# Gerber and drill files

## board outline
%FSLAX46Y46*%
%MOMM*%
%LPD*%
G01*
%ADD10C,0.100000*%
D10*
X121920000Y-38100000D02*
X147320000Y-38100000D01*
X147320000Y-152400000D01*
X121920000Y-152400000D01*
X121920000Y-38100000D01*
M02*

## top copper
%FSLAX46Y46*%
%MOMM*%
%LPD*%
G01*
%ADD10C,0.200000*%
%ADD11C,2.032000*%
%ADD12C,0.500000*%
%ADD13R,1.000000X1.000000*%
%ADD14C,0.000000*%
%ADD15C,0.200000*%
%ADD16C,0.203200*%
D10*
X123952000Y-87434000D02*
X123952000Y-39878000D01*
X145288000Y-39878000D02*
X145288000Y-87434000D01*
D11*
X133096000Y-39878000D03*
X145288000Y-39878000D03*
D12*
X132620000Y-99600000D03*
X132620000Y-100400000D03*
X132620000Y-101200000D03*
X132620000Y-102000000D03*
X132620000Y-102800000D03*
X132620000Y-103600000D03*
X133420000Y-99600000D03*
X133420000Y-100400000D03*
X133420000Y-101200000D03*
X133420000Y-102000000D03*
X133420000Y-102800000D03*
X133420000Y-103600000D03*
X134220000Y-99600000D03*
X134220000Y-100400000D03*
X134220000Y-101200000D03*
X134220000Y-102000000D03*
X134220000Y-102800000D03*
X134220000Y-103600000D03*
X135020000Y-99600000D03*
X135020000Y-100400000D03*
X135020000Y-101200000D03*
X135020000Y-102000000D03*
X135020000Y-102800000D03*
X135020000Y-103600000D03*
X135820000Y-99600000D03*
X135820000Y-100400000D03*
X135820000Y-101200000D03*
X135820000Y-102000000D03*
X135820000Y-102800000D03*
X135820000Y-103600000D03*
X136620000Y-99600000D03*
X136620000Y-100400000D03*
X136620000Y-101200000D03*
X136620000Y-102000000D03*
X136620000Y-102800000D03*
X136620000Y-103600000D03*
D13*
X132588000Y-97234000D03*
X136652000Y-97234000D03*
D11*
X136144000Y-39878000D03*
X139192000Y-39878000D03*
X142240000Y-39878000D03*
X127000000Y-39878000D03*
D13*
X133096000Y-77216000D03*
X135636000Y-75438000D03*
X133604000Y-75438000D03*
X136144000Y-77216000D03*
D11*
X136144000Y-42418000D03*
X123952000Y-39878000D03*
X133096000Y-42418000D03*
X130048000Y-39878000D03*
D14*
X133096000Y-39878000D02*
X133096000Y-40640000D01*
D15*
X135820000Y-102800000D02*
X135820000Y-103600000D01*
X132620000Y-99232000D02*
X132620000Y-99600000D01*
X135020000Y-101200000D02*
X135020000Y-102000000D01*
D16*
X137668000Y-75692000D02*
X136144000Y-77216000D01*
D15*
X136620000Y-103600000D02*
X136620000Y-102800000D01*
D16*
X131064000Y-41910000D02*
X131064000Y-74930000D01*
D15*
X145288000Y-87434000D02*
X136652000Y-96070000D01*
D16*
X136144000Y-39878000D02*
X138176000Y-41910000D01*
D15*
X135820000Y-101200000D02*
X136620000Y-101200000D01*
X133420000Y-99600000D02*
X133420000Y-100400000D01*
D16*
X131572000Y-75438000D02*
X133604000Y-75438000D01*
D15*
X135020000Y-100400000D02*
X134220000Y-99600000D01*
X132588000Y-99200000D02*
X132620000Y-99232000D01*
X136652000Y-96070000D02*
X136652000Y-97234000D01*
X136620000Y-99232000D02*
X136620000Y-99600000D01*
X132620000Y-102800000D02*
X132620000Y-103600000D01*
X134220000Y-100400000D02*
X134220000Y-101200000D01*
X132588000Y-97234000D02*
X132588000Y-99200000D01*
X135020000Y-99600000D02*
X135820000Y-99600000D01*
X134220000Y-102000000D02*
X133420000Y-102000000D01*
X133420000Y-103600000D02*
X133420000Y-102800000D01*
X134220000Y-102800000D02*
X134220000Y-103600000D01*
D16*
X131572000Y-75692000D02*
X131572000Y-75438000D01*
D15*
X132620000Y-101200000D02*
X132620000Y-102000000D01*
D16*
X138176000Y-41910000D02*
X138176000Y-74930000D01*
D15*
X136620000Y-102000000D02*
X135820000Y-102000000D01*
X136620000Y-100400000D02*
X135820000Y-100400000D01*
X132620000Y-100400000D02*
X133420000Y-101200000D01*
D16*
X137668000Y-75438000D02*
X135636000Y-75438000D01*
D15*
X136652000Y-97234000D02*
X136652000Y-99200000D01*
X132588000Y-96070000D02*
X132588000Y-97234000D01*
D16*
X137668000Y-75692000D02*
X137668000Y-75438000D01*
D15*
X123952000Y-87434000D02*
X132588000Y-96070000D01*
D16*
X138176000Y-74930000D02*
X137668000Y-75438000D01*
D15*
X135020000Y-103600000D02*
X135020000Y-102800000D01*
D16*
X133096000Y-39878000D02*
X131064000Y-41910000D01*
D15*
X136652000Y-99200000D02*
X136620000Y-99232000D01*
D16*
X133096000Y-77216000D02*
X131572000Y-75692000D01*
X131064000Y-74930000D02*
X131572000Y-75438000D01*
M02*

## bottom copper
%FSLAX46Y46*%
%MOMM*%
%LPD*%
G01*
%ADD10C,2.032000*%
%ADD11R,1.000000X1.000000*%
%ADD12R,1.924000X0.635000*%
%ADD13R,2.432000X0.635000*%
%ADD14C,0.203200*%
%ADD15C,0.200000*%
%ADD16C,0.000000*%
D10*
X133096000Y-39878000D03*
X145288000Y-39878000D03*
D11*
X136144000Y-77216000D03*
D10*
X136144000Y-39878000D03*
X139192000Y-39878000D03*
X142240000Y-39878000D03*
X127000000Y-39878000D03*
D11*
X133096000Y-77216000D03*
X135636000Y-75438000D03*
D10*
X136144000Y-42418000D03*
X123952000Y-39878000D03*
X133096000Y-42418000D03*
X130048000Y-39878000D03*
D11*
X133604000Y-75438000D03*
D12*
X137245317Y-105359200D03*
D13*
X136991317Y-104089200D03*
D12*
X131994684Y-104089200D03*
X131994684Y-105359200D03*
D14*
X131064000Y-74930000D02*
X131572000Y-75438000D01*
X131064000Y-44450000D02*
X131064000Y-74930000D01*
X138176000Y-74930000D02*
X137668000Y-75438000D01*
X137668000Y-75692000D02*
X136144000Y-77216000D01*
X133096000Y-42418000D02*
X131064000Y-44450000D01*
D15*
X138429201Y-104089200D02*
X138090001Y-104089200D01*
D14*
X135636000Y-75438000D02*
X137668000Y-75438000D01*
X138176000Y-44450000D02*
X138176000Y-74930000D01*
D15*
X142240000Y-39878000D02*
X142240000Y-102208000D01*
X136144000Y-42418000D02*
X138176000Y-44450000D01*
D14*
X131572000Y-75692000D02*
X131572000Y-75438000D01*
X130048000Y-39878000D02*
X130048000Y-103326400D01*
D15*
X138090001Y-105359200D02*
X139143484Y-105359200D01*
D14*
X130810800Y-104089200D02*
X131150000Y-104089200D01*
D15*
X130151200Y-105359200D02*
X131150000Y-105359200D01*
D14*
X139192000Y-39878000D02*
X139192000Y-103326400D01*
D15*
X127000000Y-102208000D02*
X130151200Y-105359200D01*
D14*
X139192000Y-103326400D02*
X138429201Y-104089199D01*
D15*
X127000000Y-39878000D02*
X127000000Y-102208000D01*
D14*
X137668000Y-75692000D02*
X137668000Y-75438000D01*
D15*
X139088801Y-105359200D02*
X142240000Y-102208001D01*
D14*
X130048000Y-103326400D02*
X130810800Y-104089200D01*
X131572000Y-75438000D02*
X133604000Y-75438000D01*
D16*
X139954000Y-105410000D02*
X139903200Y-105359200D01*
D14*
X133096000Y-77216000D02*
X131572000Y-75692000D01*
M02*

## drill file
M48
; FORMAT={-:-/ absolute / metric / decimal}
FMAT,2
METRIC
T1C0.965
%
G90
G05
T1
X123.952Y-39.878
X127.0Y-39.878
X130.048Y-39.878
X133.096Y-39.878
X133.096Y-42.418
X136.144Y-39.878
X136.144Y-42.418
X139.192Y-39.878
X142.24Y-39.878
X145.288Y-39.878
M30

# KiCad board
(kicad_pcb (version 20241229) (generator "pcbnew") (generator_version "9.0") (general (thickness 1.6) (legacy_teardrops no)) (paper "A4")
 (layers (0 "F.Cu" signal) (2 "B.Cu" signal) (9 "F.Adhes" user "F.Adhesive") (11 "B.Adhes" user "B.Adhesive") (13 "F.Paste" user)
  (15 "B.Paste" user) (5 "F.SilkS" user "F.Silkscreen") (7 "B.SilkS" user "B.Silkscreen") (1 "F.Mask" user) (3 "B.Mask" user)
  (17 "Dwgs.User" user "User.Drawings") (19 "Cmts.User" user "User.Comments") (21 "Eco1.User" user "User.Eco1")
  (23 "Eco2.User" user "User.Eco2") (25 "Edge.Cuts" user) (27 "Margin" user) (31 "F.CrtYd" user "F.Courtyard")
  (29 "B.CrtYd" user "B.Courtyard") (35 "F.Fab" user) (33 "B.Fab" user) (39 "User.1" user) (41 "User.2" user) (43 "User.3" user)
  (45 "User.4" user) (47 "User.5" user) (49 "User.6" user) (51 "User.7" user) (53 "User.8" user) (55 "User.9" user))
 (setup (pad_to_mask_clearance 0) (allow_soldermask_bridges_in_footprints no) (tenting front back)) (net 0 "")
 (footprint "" (layer "F.Cu") (at 133.096 52.578)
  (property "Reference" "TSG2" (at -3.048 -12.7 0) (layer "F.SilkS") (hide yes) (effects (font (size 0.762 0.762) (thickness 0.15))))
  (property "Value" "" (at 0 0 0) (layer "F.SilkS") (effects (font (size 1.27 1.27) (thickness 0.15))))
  (pad "1" thru_hole circle (at 0 -12.7) (size 2.032 2.032) (drill 0.9652) (layers "*.Cu" "*.Mask") (remove_unused_layers no)))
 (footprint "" (layer "F.Cu") (at 145.796 39.878)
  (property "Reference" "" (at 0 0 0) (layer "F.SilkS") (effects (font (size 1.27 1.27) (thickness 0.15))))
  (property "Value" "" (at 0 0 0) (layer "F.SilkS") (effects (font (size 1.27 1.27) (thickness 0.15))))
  (pad "1" thru_hole circle (at -0.508 0) (size 2.032 2.032) (drill 0.9652) (layers "*.Cu" "*.Mask") (remove_unused_layers no)))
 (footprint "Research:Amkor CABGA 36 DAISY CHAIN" (layer "F.Cu") (at 134.62 92.535)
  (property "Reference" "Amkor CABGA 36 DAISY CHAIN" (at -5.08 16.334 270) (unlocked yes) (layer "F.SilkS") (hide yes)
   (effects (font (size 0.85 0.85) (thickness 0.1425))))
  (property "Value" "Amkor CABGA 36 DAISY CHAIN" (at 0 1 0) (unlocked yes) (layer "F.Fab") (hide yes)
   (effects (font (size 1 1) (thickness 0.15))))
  (pad "1" smd circle (at -2 7.065) (size 0.5 0.5) (layers "F.Cu" "F.Mask"))
  (pad "1" smd circle (at -2 7.865) (size 0.5 0.5) (layers "F.Cu" "F.Mask"))
  (pad "1" smd circle (at -2 8.665) (size 0.5 0.5) (layers "F.Cu" "F.Mask"))
  (pad "1" smd circle (at -2 9.465) (size 0.5 0.5) (layers "F.Cu" "F.Mask"))
  (pad "1" smd circle (at -2 10.265) (size 0.5 0.5) (layers "F.Cu" "F.Mask"))
  (pad "1" smd circle (at -2 11.065) (size 0.5 0.5) (layers "F.Cu" "F.Mask"))
  (pad "1" smd circle (at -1.2 7.065) (size 0.5 0.5) (layers "F.Cu" "F.Mask"))
  (pad "1" smd circle (at -1.2 7.865) (size 0.5 0.5) (layers "F.Cu" "F.Mask"))
  (pad "1" smd circle (at -1.2 8.665) (size 0.5 0.5) (layers "F.Cu" "F.Mask"))
  (pad "1" smd circle (at -1.2 9.465) (size 0.5 0.5) (layers "F.Cu" "F.Mask"))
  (pad "1" smd circle (at -1.2 10.265) (size 0.5 0.5) (layers "F.Cu" "F.Mask"))
  (pad "1" smd circle (at -1.2 11.065) (size 0.5 0.5) (layers "F.Cu" "F.Mask"))
  (pad "1" smd circle (at -0.4 7.065) (size 0.5 0.5) (layers "F.Cu" "F.Mask"))
  (pad "1" smd circle (at -0.4 7.865) (size 0.5 0.5) (layers "F.Cu" "F.Mask"))
  (pad "1" smd circle (at -0.4 8.665) (size 0.5 0.5) (layers "F.Cu" "F.Mask"))
  (pad "1" smd circle (at -0.4 9.465) (size 0.5 0.5) (layers "F.Cu" "F.Mask"))
  (pad "1" smd circle (at -0.4 10.265) (size 0.5 0.5) (layers "F.Cu" "F.Mask"))
  (pad "1" smd circle (at -0.4 11.065) (size 0.5 0.5) (layers "F.Cu" "F.Mask"))
  (pad "1" smd circle (at 0.4 7.065) (size 0.5 0.5) (layers "F.Cu" "F.Mask"))
  (pad "1" smd circle (at 0.4 7.865) (size 0.5 0.5) (layers "F.Cu" "F.Mask"))
  (pad "1" smd circle (at 0.4 8.665) (size 0.5 0.5) (layers "F.Cu" "F.Mask"))
  (pad "1" smd circle (at 0.4 9.465) (size 0.5 0.5) (layers "F.Cu" "F.Mask"))
  (pad "1" smd circle (at 0.4 10.265) (size 0.5 0.5) (layers "F.Cu" "F.Mask"))
  (pad "1" smd circle (at 0.4 11.065) (size 0.5 0.5) (layers "F.Cu" "F.Mask"))
  (pad "1" smd circle (at 1.2 7.065) (size 0.5 0.5) (layers "F.Cu" "F.Mask"))
  (pad "1" smd circle (at 1.2 7.865) (size 0.5 0.5) (layers "F.Cu" "F.Mask"))
  (pad "1" smd circle (at 1.2 8.665) (size 0.5 0.5) (layers "F.Cu" "F.Mask"))
  (pad "1" smd circle (at 1.2 9.465) (size 0.5 0.5) (layers "F.Cu" "F.Mask"))
  (pad "1" smd circle (at 1.2 10.265) (size 0.5 0.5) (layers "F.Cu" "F.Mask"))
  (pad "1" smd circle (at 1.2 11.065) (size 0.5 0.5) (layers "F.Cu" "F.Mask"))
  (pad "1" smd circle (at 2 7.065) (size 0.5 0.5) (layers "F.Cu" "F.Mask"))
  (pad "1" smd circle (at 2 7.865) (size 0.5 0.5) (layers "F.Cu" "F.Mask"))
  (pad "1" smd circle (at 2 8.665) (size 0.5 0.5) (layers "F.Cu" "F.Mask"))
  (pad "1" smd circle (at 2 9.465) (size 0.5 0.5) (layers "F.Cu" "F.Mask"))
  (pad "1" smd circle (at 2 10.265) (size 0.5 0.5) (layers "F.Cu" "F.Mask"))
  (pad "1" smd circle (at 2 11.065) (size 0.5 0.5) (layers "F.Cu" "F.Mask"))
  (pad "2" smd rect (at -2.032 4.699) (size 1 1) (layers "F.Cu" "F.Mask"))
  (pad "3" smd rect (at 2.032 4.699) (size 1 1) (layers "F.Cu" "F.Mask")))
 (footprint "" (layer "F.Cu") (at 136.144 77.216)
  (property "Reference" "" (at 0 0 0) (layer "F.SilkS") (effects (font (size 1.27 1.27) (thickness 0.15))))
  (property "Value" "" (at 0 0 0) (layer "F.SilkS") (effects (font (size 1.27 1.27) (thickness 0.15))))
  (pad "1" smd rect (at 0 0 180) (size 1 1) (layers "B.Cu" "B.Mask")))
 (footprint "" (layer "F.Cu") (at 135.89 52.578)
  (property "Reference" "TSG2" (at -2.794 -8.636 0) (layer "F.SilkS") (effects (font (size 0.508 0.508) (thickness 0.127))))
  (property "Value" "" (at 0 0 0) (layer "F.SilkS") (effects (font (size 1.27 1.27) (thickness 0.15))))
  (pad "1" thru_hole circle (at 0.254 -12.7) (size 2.032 2.032) (drill 0.9652) (layers "*.Cu" "*.Mask") (remove_unused_layers no)))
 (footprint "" (layer "F.Cu") (at 139.192 39.878)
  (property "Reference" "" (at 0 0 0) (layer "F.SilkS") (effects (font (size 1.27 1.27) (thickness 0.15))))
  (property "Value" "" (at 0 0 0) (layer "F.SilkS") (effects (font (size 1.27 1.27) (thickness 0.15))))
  (pad "1" thru_hole circle (at 0 0) (size 2.032 2.032) (drill 0.9652) (layers "*.Cu" "*.Mask") (remove_unused_layers no)))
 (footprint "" (layer "F.Cu") (at 142.494 39.878)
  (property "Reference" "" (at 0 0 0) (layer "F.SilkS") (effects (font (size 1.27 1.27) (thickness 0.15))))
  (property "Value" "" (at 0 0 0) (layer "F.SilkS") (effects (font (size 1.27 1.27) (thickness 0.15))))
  (pad "1" thru_hole circle (at -0.254 0) (size 2.032 2.032) (drill 0.9652) (layers "*.Cu" "*.Mask") (remove_unused_layers no)))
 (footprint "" (layer "F.Cu") (at 127 39.878)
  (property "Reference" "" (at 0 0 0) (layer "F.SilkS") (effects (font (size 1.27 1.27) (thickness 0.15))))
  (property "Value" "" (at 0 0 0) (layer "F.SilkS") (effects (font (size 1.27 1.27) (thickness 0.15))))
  (pad "1" thru_hole circle (at 0 0) (size 2.032 2.032) (drill 0.9652) (layers "*.Cu" "*.Mask") (remove_unused_layers no)))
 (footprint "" (layer "F.Cu") (at 133.096 77.216)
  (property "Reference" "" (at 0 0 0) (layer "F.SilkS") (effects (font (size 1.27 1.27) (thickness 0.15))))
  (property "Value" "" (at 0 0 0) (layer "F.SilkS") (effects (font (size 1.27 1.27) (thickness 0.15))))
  (pad "1" smd rect (at 0 0) (size 1 1) (layers "F.Cu" "F.Mask")))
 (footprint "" (layer "F.Cu") (at 133.096 77.216)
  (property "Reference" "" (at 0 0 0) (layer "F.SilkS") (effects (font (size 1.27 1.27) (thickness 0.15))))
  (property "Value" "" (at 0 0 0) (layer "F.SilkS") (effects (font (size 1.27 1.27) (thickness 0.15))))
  (pad "1" smd rect (at 0 0 180) (size 1 1) (layers "B.Cu" "B.Mask")))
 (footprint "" (layer "F.Cu") (at 135.636 75.438)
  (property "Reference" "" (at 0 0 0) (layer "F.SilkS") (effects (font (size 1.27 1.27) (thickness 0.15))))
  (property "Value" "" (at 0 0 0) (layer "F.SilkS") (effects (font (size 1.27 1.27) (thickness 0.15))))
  (pad "1" smd rect (at 0 0) (size 1 1) (layers "F.Cu" "F.Mask")))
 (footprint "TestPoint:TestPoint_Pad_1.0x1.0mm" (layer "F.Cu") (at 133.604 75.438)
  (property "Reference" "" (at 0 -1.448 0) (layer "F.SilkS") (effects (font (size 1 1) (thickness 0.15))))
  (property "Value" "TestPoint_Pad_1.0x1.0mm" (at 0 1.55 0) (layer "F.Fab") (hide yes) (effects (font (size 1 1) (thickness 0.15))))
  (pad "1" smd rect (at 0 0) (size 1 1) (layers "F.Cu" "F.Mask")))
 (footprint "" (layer "F.Cu") (at 136.144 77.216)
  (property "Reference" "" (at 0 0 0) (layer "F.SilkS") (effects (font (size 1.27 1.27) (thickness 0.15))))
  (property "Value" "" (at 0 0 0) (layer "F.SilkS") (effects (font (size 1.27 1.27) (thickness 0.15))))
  (pad "1" smd rect (at 0 0) (size 1 1) (layers "F.Cu" "F.Mask")))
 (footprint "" (layer "F.Cu") (at 135.636 75.438)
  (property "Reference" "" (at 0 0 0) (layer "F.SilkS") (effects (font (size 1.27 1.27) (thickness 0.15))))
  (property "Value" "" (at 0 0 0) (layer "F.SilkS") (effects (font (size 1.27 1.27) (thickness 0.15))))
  (pad "1" smd rect (at 0 0 180) (size 1 1) (layers "B.Cu" "B.Mask")))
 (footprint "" (layer "F.Cu") (at 135.89 55.118)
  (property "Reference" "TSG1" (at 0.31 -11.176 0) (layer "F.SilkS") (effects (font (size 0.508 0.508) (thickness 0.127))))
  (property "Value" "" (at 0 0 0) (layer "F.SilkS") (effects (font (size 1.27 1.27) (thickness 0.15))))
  (pad "1" thru_hole circle (at 0.254 -12.7) (size 2.032 2.032) (drill 0.9652) (layers "*.Cu" "*.Mask") (remove_unused_layers no)))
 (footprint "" (layer "F.Cu") (at 123.952 39.878)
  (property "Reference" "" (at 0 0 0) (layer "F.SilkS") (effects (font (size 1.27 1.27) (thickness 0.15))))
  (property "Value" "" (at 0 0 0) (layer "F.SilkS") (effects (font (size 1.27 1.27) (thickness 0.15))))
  (pad "1" thru_hole circle (at 0 0) (size 2.032 2.032) (drill 0.9652) (layers "*.Cu" "*.Mask") (remove_unused_layers no)))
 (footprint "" (layer "F.Cu") (at 133.096 55.118)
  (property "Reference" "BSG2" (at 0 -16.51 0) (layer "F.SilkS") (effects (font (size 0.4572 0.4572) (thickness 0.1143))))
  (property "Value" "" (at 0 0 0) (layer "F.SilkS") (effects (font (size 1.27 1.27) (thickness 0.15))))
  (pad "1" thru_hole circle (at 0 -12.7) (size 2.032 2.032) (drill 0.9652) (layers "*.Cu" "*.Mask") (remove_unused_layers no)))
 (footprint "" (layer "B.Cu") (at 130.048 39.878)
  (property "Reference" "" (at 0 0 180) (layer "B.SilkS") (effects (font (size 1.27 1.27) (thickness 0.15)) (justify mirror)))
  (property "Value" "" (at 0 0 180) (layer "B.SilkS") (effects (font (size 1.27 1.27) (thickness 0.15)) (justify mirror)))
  (pad "1" thru_hole circle (at 0 0) (size 2.032 2.032) (drill 0.9652) (layers "*.Cu" "*.Mask") (remove_unused_layers no)))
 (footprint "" (layer "B.Cu") (at 133.604 75.438 180)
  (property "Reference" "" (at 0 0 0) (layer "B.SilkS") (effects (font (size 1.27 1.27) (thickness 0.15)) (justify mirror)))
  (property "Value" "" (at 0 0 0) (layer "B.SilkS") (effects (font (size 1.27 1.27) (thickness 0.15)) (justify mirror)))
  (pad "1" smd rect (at 0 0 180) (size 1 1) (layers "B.Cu" "B.Mask")))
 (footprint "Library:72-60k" (layer "B.Cu") (at 132.873329 109.1692 180)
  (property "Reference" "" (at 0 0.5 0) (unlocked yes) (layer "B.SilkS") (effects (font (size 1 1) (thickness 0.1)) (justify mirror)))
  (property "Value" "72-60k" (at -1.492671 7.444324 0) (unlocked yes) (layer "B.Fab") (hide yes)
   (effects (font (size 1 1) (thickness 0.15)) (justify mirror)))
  (pad "1" smd rect (at -4.371988 3.81) (size 1.924 0.635) (layers "B.Cu" "B.Mask"))
  (pad "2" smd rect (at -4.117988 5.08) (size 2.432 0.635) (layers "B.Cu" "B.Mask"))
  (pad "3" smd rect (at 0.878645 5.08) (size 1.924 0.635) (layers "B.Cu" "B.Mask"))
  (pad "4" smd rect (at 0.878645 3.81) (size 1.924 0.635) (layers "B.Cu" "B.Mask")))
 (gr_line (start 123.952 87.434) (end 123.952 39.878) (stroke (width 0.2) (type solid)) (layer "F.Cu"))
 (gr_line (start 145.288 39.878) (end 145.288 87.434) (stroke (width 0.2) (type solid)) (layer "F.Cu"))
 (gr_rect (start 121.92 38.1) (end 147.32 152.4) (stroke (width 0.1) (type solid)) (fill no) (layer "Edge.Cuts"))
 (segment (start 133.096 39.878) (end 133.096 40.64) (width 0) (layer "F.Cu") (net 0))
 (segment (start 135.82 102.8) (end 135.82 103.6) (width 0.2) (layer "F.Cu") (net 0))
 (segment (start 132.62 99.232) (end 132.62 99.6) (width 0.2) (layer "F.Cu") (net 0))
 (segment (start 135.02 101.2) (end 135.02 102) (width 0.2) (layer "F.Cu") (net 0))
 (segment (start 137.668 75.692) (end 136.144 77.216) (width 0.2032) (layer "F.Cu") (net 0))
 (segment (start 136.62 103.6) (end 136.62 102.8) (width 0.2) (layer "F.Cu") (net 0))
 (segment (start 131.064 41.91) (end 131.064 74.93) (width 0.2032) (layer "F.Cu") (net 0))
 (segment (start 145.288 87.434) (end 136.652 96.07) (width 0.2) (layer "F.Cu") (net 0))
 (segment (start 136.144 39.878) (end 138.176 41.91) (width 0.2032) (layer "F.Cu") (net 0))
 (segment (start 135.82 101.2) (end 136.62 101.2) (width 0.2) (layer "F.Cu") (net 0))
 (segment (start 133.42 99.6) (end 133.42 100.4) (width 0.2) (layer "F.Cu") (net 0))
 (segment (start 131.572 75.438) (end 133.604 75.438) (width 0.2032) (layer "F.Cu") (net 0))
 (segment (start 135.02 100.4) (end 134.22 99.6) (width 0.2) (layer "F.Cu") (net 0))
 (segment (start 132.588 99.2) (end 132.62 99.232) (width 0.2) (layer "F.Cu") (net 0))
 (segment (start 136.652 96.07) (end 136.652 97.234) (width 0.2) (layer "F.Cu") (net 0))
 (segment (start 136.62 99.232) (end 136.62 99.6) (width 0.2) (layer "F.Cu") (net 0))
 (segment (start 132.62 102.8) (end 132.62 103.6) (width 0.2) (layer "F.Cu") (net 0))
 (segment (start 134.22 100.4) (end 134.22 101.2) (width 0.2) (layer "F.Cu") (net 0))
 (segment (start 132.588 97.234) (end 132.588 99.2) (width 0.2) (layer "F.Cu") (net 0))
 (segment (start 135.02 99.6) (end 135.82 99.6) (width 0.2) (layer "F.Cu") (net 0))
 (segment (start 134.22 102) (end 133.42 102) (width 0.2) (layer "F.Cu") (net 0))
 (segment (start 133.42 103.6) (end 133.42 102.8) (width 0.2) (layer "F.Cu") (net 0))
 (segment (start 134.22 102.8) (end 134.22 103.6) (width 0.2) (layer "F.Cu") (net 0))
 (segment (start 131.572 75.692) (end 131.572 75.438) (width 0.2032) (layer "F.Cu") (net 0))
 (segment (start 132.62 101.2) (end 132.62 102) (width 0.2) (layer "F.Cu") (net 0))
 (segment (start 138.176 41.91) (end 138.176 74.93) (width 0.2032) (layer "F.Cu") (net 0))
 (segment (start 136.62 102) (end 135.82 102) (width 0.2) (layer "F.Cu") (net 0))
 (segment (start 136.62 100.4) (end 135.82 100.4) (width 0.2) (layer "F.Cu") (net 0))
 (segment (start 132.62 100.4) (end 133.42 101.2) (width 0.2) (layer "F.Cu") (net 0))
 (segment (start 137.668 75.438) (end 135.636 75.438) (width 0.2032) (layer "F.Cu") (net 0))
 (segment (start 136.652 97.234) (end 136.652 99.2) (width 0.2) (layer "F.Cu") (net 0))
 (segment (start 132.588 96.07) (end 132.588 97.234) (width 0.2) (layer "F.Cu") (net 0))
 (segment (start 137.668 75.692) (end 137.668 75.438) (width 0.2032) (layer "F.Cu") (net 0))
 (segment (start 123.952 87.434) (end 132.588 96.07) (width 0.2) (layer "F.Cu") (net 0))
 (segment (start 138.176 74.93) (end 137.668 75.438) (width 0.2032) (layer "F.Cu") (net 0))
 (segment (start 135.02 103.6) (end 135.02 102.8) (width 0.2) (layer "F.Cu") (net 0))
 (segment (start 133.096 39.878) (end 131.064 41.91) (width 0.2032) (layer "F.Cu") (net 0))
 (segment (start 136.652 99.2) (end 136.62 99.232) (width 0.2) (layer "F.Cu") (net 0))
 (segment (start 133.096 77.216) (end 131.572 75.692) (width 0.2032) (layer "F.Cu") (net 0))
 (segment (start 131.064 74.93) (end 131.572 75.438) (width 0.2032) (layer "F.Cu") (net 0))
 (segment (start 131.064 74.93) (end 131.572 75.438) (width 0.2032) (layer "B.Cu") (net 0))
 (segment (start 131.064 44.45) (end 131.064 74.93) (width 0.2032) (layer "B.Cu") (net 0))
 (segment (start 138.176 74.93) (end 137.668 75.438) (width 0.2032) (layer "B.Cu") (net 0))
 (segment (start 137.668 75.692) (end 136.144 77.216) (width 0.2032) (layer "B.Cu") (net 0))
 (segment (start 133.096 42.418) (end 131.064 44.45) (width 0.2032) (layer "B.Cu") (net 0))
 (segment (start 138.429201 104.0892) (end 138.090001 104.0892) (width 0.2) (layer "B.Cu") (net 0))
 (segment (start 135.636 75.438) (end 137.668 75.438) (width 0.2032) (layer "B.Cu") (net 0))
 (segment (start 138.176 44.45) (end 138.176 74.93) (width 0.2032) (layer "B.Cu") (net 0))
 (segment (start 142.24 39.878) (end 142.24 102.208) (width 0.2) (layer "B.Cu") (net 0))
 (segment (start 136.144 42.418) (end 138.176 44.45) (width 0.2) (layer "B.Cu") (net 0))
 (segment (start 131.572 75.692) (end 131.572 75.438) (width 0.2032) (layer "B.Cu") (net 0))
 (segment (start 130.048 39.878) (end 130.048 103.3264) (width 0.2032) (layer "B.Cu") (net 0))
 (segment (start 138.090001 105.3592) (end 139.143484 105.3592) (width 0.2) (layer "B.Cu") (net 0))
 (segment (start 130.8108 104.0892) (end 131.15 104.0892) (width 0.2032) (layer "B.Cu") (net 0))
 (segment (start 130.1512 105.3592) (end 131.15 105.3592) (width 0.2) (layer "B.Cu") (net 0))
 (segment (start 139.192 39.878) (end 139.192 103.3264) (width 0.2032) (layer "B.Cu") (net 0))
 (segment (start 127 102.208) (end 130.1512 105.3592) (width 0.2) (layer "B.Cu") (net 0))
 (segment (start 139.192 103.3264) (end 138.429201 104.089199) (width 0.2032) (layer "B.Cu") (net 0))
 (segment (start 127 39.878) (end 127 102.208) (width 0.2) (layer "B.Cu") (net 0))
 (segment (start 137.668 75.692) (end 137.668 75.438) (width 0.2032) (layer "B.Cu") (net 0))
 (segment (start 139.088801 105.3592) (end 142.24 102.208001) (width 0.2) (layer "B.Cu") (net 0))
 (segment (start 130.048 103.3264) (end 130.8108 104.0892) (width 0.2032) (layer "B.Cu") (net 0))
 (segment (start 131.572 75.438) (end 133.604 75.438) (width 0.2032) (layer "B.Cu") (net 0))
 (segment (start 139.954 105.41) (end 139.9032 105.3592) (width 0) (layer "B.Cu") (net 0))
 (segment (start 133.096 77.216) (end 131.572 75.692) (width 0.2032) (layer "B.Cu") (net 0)))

